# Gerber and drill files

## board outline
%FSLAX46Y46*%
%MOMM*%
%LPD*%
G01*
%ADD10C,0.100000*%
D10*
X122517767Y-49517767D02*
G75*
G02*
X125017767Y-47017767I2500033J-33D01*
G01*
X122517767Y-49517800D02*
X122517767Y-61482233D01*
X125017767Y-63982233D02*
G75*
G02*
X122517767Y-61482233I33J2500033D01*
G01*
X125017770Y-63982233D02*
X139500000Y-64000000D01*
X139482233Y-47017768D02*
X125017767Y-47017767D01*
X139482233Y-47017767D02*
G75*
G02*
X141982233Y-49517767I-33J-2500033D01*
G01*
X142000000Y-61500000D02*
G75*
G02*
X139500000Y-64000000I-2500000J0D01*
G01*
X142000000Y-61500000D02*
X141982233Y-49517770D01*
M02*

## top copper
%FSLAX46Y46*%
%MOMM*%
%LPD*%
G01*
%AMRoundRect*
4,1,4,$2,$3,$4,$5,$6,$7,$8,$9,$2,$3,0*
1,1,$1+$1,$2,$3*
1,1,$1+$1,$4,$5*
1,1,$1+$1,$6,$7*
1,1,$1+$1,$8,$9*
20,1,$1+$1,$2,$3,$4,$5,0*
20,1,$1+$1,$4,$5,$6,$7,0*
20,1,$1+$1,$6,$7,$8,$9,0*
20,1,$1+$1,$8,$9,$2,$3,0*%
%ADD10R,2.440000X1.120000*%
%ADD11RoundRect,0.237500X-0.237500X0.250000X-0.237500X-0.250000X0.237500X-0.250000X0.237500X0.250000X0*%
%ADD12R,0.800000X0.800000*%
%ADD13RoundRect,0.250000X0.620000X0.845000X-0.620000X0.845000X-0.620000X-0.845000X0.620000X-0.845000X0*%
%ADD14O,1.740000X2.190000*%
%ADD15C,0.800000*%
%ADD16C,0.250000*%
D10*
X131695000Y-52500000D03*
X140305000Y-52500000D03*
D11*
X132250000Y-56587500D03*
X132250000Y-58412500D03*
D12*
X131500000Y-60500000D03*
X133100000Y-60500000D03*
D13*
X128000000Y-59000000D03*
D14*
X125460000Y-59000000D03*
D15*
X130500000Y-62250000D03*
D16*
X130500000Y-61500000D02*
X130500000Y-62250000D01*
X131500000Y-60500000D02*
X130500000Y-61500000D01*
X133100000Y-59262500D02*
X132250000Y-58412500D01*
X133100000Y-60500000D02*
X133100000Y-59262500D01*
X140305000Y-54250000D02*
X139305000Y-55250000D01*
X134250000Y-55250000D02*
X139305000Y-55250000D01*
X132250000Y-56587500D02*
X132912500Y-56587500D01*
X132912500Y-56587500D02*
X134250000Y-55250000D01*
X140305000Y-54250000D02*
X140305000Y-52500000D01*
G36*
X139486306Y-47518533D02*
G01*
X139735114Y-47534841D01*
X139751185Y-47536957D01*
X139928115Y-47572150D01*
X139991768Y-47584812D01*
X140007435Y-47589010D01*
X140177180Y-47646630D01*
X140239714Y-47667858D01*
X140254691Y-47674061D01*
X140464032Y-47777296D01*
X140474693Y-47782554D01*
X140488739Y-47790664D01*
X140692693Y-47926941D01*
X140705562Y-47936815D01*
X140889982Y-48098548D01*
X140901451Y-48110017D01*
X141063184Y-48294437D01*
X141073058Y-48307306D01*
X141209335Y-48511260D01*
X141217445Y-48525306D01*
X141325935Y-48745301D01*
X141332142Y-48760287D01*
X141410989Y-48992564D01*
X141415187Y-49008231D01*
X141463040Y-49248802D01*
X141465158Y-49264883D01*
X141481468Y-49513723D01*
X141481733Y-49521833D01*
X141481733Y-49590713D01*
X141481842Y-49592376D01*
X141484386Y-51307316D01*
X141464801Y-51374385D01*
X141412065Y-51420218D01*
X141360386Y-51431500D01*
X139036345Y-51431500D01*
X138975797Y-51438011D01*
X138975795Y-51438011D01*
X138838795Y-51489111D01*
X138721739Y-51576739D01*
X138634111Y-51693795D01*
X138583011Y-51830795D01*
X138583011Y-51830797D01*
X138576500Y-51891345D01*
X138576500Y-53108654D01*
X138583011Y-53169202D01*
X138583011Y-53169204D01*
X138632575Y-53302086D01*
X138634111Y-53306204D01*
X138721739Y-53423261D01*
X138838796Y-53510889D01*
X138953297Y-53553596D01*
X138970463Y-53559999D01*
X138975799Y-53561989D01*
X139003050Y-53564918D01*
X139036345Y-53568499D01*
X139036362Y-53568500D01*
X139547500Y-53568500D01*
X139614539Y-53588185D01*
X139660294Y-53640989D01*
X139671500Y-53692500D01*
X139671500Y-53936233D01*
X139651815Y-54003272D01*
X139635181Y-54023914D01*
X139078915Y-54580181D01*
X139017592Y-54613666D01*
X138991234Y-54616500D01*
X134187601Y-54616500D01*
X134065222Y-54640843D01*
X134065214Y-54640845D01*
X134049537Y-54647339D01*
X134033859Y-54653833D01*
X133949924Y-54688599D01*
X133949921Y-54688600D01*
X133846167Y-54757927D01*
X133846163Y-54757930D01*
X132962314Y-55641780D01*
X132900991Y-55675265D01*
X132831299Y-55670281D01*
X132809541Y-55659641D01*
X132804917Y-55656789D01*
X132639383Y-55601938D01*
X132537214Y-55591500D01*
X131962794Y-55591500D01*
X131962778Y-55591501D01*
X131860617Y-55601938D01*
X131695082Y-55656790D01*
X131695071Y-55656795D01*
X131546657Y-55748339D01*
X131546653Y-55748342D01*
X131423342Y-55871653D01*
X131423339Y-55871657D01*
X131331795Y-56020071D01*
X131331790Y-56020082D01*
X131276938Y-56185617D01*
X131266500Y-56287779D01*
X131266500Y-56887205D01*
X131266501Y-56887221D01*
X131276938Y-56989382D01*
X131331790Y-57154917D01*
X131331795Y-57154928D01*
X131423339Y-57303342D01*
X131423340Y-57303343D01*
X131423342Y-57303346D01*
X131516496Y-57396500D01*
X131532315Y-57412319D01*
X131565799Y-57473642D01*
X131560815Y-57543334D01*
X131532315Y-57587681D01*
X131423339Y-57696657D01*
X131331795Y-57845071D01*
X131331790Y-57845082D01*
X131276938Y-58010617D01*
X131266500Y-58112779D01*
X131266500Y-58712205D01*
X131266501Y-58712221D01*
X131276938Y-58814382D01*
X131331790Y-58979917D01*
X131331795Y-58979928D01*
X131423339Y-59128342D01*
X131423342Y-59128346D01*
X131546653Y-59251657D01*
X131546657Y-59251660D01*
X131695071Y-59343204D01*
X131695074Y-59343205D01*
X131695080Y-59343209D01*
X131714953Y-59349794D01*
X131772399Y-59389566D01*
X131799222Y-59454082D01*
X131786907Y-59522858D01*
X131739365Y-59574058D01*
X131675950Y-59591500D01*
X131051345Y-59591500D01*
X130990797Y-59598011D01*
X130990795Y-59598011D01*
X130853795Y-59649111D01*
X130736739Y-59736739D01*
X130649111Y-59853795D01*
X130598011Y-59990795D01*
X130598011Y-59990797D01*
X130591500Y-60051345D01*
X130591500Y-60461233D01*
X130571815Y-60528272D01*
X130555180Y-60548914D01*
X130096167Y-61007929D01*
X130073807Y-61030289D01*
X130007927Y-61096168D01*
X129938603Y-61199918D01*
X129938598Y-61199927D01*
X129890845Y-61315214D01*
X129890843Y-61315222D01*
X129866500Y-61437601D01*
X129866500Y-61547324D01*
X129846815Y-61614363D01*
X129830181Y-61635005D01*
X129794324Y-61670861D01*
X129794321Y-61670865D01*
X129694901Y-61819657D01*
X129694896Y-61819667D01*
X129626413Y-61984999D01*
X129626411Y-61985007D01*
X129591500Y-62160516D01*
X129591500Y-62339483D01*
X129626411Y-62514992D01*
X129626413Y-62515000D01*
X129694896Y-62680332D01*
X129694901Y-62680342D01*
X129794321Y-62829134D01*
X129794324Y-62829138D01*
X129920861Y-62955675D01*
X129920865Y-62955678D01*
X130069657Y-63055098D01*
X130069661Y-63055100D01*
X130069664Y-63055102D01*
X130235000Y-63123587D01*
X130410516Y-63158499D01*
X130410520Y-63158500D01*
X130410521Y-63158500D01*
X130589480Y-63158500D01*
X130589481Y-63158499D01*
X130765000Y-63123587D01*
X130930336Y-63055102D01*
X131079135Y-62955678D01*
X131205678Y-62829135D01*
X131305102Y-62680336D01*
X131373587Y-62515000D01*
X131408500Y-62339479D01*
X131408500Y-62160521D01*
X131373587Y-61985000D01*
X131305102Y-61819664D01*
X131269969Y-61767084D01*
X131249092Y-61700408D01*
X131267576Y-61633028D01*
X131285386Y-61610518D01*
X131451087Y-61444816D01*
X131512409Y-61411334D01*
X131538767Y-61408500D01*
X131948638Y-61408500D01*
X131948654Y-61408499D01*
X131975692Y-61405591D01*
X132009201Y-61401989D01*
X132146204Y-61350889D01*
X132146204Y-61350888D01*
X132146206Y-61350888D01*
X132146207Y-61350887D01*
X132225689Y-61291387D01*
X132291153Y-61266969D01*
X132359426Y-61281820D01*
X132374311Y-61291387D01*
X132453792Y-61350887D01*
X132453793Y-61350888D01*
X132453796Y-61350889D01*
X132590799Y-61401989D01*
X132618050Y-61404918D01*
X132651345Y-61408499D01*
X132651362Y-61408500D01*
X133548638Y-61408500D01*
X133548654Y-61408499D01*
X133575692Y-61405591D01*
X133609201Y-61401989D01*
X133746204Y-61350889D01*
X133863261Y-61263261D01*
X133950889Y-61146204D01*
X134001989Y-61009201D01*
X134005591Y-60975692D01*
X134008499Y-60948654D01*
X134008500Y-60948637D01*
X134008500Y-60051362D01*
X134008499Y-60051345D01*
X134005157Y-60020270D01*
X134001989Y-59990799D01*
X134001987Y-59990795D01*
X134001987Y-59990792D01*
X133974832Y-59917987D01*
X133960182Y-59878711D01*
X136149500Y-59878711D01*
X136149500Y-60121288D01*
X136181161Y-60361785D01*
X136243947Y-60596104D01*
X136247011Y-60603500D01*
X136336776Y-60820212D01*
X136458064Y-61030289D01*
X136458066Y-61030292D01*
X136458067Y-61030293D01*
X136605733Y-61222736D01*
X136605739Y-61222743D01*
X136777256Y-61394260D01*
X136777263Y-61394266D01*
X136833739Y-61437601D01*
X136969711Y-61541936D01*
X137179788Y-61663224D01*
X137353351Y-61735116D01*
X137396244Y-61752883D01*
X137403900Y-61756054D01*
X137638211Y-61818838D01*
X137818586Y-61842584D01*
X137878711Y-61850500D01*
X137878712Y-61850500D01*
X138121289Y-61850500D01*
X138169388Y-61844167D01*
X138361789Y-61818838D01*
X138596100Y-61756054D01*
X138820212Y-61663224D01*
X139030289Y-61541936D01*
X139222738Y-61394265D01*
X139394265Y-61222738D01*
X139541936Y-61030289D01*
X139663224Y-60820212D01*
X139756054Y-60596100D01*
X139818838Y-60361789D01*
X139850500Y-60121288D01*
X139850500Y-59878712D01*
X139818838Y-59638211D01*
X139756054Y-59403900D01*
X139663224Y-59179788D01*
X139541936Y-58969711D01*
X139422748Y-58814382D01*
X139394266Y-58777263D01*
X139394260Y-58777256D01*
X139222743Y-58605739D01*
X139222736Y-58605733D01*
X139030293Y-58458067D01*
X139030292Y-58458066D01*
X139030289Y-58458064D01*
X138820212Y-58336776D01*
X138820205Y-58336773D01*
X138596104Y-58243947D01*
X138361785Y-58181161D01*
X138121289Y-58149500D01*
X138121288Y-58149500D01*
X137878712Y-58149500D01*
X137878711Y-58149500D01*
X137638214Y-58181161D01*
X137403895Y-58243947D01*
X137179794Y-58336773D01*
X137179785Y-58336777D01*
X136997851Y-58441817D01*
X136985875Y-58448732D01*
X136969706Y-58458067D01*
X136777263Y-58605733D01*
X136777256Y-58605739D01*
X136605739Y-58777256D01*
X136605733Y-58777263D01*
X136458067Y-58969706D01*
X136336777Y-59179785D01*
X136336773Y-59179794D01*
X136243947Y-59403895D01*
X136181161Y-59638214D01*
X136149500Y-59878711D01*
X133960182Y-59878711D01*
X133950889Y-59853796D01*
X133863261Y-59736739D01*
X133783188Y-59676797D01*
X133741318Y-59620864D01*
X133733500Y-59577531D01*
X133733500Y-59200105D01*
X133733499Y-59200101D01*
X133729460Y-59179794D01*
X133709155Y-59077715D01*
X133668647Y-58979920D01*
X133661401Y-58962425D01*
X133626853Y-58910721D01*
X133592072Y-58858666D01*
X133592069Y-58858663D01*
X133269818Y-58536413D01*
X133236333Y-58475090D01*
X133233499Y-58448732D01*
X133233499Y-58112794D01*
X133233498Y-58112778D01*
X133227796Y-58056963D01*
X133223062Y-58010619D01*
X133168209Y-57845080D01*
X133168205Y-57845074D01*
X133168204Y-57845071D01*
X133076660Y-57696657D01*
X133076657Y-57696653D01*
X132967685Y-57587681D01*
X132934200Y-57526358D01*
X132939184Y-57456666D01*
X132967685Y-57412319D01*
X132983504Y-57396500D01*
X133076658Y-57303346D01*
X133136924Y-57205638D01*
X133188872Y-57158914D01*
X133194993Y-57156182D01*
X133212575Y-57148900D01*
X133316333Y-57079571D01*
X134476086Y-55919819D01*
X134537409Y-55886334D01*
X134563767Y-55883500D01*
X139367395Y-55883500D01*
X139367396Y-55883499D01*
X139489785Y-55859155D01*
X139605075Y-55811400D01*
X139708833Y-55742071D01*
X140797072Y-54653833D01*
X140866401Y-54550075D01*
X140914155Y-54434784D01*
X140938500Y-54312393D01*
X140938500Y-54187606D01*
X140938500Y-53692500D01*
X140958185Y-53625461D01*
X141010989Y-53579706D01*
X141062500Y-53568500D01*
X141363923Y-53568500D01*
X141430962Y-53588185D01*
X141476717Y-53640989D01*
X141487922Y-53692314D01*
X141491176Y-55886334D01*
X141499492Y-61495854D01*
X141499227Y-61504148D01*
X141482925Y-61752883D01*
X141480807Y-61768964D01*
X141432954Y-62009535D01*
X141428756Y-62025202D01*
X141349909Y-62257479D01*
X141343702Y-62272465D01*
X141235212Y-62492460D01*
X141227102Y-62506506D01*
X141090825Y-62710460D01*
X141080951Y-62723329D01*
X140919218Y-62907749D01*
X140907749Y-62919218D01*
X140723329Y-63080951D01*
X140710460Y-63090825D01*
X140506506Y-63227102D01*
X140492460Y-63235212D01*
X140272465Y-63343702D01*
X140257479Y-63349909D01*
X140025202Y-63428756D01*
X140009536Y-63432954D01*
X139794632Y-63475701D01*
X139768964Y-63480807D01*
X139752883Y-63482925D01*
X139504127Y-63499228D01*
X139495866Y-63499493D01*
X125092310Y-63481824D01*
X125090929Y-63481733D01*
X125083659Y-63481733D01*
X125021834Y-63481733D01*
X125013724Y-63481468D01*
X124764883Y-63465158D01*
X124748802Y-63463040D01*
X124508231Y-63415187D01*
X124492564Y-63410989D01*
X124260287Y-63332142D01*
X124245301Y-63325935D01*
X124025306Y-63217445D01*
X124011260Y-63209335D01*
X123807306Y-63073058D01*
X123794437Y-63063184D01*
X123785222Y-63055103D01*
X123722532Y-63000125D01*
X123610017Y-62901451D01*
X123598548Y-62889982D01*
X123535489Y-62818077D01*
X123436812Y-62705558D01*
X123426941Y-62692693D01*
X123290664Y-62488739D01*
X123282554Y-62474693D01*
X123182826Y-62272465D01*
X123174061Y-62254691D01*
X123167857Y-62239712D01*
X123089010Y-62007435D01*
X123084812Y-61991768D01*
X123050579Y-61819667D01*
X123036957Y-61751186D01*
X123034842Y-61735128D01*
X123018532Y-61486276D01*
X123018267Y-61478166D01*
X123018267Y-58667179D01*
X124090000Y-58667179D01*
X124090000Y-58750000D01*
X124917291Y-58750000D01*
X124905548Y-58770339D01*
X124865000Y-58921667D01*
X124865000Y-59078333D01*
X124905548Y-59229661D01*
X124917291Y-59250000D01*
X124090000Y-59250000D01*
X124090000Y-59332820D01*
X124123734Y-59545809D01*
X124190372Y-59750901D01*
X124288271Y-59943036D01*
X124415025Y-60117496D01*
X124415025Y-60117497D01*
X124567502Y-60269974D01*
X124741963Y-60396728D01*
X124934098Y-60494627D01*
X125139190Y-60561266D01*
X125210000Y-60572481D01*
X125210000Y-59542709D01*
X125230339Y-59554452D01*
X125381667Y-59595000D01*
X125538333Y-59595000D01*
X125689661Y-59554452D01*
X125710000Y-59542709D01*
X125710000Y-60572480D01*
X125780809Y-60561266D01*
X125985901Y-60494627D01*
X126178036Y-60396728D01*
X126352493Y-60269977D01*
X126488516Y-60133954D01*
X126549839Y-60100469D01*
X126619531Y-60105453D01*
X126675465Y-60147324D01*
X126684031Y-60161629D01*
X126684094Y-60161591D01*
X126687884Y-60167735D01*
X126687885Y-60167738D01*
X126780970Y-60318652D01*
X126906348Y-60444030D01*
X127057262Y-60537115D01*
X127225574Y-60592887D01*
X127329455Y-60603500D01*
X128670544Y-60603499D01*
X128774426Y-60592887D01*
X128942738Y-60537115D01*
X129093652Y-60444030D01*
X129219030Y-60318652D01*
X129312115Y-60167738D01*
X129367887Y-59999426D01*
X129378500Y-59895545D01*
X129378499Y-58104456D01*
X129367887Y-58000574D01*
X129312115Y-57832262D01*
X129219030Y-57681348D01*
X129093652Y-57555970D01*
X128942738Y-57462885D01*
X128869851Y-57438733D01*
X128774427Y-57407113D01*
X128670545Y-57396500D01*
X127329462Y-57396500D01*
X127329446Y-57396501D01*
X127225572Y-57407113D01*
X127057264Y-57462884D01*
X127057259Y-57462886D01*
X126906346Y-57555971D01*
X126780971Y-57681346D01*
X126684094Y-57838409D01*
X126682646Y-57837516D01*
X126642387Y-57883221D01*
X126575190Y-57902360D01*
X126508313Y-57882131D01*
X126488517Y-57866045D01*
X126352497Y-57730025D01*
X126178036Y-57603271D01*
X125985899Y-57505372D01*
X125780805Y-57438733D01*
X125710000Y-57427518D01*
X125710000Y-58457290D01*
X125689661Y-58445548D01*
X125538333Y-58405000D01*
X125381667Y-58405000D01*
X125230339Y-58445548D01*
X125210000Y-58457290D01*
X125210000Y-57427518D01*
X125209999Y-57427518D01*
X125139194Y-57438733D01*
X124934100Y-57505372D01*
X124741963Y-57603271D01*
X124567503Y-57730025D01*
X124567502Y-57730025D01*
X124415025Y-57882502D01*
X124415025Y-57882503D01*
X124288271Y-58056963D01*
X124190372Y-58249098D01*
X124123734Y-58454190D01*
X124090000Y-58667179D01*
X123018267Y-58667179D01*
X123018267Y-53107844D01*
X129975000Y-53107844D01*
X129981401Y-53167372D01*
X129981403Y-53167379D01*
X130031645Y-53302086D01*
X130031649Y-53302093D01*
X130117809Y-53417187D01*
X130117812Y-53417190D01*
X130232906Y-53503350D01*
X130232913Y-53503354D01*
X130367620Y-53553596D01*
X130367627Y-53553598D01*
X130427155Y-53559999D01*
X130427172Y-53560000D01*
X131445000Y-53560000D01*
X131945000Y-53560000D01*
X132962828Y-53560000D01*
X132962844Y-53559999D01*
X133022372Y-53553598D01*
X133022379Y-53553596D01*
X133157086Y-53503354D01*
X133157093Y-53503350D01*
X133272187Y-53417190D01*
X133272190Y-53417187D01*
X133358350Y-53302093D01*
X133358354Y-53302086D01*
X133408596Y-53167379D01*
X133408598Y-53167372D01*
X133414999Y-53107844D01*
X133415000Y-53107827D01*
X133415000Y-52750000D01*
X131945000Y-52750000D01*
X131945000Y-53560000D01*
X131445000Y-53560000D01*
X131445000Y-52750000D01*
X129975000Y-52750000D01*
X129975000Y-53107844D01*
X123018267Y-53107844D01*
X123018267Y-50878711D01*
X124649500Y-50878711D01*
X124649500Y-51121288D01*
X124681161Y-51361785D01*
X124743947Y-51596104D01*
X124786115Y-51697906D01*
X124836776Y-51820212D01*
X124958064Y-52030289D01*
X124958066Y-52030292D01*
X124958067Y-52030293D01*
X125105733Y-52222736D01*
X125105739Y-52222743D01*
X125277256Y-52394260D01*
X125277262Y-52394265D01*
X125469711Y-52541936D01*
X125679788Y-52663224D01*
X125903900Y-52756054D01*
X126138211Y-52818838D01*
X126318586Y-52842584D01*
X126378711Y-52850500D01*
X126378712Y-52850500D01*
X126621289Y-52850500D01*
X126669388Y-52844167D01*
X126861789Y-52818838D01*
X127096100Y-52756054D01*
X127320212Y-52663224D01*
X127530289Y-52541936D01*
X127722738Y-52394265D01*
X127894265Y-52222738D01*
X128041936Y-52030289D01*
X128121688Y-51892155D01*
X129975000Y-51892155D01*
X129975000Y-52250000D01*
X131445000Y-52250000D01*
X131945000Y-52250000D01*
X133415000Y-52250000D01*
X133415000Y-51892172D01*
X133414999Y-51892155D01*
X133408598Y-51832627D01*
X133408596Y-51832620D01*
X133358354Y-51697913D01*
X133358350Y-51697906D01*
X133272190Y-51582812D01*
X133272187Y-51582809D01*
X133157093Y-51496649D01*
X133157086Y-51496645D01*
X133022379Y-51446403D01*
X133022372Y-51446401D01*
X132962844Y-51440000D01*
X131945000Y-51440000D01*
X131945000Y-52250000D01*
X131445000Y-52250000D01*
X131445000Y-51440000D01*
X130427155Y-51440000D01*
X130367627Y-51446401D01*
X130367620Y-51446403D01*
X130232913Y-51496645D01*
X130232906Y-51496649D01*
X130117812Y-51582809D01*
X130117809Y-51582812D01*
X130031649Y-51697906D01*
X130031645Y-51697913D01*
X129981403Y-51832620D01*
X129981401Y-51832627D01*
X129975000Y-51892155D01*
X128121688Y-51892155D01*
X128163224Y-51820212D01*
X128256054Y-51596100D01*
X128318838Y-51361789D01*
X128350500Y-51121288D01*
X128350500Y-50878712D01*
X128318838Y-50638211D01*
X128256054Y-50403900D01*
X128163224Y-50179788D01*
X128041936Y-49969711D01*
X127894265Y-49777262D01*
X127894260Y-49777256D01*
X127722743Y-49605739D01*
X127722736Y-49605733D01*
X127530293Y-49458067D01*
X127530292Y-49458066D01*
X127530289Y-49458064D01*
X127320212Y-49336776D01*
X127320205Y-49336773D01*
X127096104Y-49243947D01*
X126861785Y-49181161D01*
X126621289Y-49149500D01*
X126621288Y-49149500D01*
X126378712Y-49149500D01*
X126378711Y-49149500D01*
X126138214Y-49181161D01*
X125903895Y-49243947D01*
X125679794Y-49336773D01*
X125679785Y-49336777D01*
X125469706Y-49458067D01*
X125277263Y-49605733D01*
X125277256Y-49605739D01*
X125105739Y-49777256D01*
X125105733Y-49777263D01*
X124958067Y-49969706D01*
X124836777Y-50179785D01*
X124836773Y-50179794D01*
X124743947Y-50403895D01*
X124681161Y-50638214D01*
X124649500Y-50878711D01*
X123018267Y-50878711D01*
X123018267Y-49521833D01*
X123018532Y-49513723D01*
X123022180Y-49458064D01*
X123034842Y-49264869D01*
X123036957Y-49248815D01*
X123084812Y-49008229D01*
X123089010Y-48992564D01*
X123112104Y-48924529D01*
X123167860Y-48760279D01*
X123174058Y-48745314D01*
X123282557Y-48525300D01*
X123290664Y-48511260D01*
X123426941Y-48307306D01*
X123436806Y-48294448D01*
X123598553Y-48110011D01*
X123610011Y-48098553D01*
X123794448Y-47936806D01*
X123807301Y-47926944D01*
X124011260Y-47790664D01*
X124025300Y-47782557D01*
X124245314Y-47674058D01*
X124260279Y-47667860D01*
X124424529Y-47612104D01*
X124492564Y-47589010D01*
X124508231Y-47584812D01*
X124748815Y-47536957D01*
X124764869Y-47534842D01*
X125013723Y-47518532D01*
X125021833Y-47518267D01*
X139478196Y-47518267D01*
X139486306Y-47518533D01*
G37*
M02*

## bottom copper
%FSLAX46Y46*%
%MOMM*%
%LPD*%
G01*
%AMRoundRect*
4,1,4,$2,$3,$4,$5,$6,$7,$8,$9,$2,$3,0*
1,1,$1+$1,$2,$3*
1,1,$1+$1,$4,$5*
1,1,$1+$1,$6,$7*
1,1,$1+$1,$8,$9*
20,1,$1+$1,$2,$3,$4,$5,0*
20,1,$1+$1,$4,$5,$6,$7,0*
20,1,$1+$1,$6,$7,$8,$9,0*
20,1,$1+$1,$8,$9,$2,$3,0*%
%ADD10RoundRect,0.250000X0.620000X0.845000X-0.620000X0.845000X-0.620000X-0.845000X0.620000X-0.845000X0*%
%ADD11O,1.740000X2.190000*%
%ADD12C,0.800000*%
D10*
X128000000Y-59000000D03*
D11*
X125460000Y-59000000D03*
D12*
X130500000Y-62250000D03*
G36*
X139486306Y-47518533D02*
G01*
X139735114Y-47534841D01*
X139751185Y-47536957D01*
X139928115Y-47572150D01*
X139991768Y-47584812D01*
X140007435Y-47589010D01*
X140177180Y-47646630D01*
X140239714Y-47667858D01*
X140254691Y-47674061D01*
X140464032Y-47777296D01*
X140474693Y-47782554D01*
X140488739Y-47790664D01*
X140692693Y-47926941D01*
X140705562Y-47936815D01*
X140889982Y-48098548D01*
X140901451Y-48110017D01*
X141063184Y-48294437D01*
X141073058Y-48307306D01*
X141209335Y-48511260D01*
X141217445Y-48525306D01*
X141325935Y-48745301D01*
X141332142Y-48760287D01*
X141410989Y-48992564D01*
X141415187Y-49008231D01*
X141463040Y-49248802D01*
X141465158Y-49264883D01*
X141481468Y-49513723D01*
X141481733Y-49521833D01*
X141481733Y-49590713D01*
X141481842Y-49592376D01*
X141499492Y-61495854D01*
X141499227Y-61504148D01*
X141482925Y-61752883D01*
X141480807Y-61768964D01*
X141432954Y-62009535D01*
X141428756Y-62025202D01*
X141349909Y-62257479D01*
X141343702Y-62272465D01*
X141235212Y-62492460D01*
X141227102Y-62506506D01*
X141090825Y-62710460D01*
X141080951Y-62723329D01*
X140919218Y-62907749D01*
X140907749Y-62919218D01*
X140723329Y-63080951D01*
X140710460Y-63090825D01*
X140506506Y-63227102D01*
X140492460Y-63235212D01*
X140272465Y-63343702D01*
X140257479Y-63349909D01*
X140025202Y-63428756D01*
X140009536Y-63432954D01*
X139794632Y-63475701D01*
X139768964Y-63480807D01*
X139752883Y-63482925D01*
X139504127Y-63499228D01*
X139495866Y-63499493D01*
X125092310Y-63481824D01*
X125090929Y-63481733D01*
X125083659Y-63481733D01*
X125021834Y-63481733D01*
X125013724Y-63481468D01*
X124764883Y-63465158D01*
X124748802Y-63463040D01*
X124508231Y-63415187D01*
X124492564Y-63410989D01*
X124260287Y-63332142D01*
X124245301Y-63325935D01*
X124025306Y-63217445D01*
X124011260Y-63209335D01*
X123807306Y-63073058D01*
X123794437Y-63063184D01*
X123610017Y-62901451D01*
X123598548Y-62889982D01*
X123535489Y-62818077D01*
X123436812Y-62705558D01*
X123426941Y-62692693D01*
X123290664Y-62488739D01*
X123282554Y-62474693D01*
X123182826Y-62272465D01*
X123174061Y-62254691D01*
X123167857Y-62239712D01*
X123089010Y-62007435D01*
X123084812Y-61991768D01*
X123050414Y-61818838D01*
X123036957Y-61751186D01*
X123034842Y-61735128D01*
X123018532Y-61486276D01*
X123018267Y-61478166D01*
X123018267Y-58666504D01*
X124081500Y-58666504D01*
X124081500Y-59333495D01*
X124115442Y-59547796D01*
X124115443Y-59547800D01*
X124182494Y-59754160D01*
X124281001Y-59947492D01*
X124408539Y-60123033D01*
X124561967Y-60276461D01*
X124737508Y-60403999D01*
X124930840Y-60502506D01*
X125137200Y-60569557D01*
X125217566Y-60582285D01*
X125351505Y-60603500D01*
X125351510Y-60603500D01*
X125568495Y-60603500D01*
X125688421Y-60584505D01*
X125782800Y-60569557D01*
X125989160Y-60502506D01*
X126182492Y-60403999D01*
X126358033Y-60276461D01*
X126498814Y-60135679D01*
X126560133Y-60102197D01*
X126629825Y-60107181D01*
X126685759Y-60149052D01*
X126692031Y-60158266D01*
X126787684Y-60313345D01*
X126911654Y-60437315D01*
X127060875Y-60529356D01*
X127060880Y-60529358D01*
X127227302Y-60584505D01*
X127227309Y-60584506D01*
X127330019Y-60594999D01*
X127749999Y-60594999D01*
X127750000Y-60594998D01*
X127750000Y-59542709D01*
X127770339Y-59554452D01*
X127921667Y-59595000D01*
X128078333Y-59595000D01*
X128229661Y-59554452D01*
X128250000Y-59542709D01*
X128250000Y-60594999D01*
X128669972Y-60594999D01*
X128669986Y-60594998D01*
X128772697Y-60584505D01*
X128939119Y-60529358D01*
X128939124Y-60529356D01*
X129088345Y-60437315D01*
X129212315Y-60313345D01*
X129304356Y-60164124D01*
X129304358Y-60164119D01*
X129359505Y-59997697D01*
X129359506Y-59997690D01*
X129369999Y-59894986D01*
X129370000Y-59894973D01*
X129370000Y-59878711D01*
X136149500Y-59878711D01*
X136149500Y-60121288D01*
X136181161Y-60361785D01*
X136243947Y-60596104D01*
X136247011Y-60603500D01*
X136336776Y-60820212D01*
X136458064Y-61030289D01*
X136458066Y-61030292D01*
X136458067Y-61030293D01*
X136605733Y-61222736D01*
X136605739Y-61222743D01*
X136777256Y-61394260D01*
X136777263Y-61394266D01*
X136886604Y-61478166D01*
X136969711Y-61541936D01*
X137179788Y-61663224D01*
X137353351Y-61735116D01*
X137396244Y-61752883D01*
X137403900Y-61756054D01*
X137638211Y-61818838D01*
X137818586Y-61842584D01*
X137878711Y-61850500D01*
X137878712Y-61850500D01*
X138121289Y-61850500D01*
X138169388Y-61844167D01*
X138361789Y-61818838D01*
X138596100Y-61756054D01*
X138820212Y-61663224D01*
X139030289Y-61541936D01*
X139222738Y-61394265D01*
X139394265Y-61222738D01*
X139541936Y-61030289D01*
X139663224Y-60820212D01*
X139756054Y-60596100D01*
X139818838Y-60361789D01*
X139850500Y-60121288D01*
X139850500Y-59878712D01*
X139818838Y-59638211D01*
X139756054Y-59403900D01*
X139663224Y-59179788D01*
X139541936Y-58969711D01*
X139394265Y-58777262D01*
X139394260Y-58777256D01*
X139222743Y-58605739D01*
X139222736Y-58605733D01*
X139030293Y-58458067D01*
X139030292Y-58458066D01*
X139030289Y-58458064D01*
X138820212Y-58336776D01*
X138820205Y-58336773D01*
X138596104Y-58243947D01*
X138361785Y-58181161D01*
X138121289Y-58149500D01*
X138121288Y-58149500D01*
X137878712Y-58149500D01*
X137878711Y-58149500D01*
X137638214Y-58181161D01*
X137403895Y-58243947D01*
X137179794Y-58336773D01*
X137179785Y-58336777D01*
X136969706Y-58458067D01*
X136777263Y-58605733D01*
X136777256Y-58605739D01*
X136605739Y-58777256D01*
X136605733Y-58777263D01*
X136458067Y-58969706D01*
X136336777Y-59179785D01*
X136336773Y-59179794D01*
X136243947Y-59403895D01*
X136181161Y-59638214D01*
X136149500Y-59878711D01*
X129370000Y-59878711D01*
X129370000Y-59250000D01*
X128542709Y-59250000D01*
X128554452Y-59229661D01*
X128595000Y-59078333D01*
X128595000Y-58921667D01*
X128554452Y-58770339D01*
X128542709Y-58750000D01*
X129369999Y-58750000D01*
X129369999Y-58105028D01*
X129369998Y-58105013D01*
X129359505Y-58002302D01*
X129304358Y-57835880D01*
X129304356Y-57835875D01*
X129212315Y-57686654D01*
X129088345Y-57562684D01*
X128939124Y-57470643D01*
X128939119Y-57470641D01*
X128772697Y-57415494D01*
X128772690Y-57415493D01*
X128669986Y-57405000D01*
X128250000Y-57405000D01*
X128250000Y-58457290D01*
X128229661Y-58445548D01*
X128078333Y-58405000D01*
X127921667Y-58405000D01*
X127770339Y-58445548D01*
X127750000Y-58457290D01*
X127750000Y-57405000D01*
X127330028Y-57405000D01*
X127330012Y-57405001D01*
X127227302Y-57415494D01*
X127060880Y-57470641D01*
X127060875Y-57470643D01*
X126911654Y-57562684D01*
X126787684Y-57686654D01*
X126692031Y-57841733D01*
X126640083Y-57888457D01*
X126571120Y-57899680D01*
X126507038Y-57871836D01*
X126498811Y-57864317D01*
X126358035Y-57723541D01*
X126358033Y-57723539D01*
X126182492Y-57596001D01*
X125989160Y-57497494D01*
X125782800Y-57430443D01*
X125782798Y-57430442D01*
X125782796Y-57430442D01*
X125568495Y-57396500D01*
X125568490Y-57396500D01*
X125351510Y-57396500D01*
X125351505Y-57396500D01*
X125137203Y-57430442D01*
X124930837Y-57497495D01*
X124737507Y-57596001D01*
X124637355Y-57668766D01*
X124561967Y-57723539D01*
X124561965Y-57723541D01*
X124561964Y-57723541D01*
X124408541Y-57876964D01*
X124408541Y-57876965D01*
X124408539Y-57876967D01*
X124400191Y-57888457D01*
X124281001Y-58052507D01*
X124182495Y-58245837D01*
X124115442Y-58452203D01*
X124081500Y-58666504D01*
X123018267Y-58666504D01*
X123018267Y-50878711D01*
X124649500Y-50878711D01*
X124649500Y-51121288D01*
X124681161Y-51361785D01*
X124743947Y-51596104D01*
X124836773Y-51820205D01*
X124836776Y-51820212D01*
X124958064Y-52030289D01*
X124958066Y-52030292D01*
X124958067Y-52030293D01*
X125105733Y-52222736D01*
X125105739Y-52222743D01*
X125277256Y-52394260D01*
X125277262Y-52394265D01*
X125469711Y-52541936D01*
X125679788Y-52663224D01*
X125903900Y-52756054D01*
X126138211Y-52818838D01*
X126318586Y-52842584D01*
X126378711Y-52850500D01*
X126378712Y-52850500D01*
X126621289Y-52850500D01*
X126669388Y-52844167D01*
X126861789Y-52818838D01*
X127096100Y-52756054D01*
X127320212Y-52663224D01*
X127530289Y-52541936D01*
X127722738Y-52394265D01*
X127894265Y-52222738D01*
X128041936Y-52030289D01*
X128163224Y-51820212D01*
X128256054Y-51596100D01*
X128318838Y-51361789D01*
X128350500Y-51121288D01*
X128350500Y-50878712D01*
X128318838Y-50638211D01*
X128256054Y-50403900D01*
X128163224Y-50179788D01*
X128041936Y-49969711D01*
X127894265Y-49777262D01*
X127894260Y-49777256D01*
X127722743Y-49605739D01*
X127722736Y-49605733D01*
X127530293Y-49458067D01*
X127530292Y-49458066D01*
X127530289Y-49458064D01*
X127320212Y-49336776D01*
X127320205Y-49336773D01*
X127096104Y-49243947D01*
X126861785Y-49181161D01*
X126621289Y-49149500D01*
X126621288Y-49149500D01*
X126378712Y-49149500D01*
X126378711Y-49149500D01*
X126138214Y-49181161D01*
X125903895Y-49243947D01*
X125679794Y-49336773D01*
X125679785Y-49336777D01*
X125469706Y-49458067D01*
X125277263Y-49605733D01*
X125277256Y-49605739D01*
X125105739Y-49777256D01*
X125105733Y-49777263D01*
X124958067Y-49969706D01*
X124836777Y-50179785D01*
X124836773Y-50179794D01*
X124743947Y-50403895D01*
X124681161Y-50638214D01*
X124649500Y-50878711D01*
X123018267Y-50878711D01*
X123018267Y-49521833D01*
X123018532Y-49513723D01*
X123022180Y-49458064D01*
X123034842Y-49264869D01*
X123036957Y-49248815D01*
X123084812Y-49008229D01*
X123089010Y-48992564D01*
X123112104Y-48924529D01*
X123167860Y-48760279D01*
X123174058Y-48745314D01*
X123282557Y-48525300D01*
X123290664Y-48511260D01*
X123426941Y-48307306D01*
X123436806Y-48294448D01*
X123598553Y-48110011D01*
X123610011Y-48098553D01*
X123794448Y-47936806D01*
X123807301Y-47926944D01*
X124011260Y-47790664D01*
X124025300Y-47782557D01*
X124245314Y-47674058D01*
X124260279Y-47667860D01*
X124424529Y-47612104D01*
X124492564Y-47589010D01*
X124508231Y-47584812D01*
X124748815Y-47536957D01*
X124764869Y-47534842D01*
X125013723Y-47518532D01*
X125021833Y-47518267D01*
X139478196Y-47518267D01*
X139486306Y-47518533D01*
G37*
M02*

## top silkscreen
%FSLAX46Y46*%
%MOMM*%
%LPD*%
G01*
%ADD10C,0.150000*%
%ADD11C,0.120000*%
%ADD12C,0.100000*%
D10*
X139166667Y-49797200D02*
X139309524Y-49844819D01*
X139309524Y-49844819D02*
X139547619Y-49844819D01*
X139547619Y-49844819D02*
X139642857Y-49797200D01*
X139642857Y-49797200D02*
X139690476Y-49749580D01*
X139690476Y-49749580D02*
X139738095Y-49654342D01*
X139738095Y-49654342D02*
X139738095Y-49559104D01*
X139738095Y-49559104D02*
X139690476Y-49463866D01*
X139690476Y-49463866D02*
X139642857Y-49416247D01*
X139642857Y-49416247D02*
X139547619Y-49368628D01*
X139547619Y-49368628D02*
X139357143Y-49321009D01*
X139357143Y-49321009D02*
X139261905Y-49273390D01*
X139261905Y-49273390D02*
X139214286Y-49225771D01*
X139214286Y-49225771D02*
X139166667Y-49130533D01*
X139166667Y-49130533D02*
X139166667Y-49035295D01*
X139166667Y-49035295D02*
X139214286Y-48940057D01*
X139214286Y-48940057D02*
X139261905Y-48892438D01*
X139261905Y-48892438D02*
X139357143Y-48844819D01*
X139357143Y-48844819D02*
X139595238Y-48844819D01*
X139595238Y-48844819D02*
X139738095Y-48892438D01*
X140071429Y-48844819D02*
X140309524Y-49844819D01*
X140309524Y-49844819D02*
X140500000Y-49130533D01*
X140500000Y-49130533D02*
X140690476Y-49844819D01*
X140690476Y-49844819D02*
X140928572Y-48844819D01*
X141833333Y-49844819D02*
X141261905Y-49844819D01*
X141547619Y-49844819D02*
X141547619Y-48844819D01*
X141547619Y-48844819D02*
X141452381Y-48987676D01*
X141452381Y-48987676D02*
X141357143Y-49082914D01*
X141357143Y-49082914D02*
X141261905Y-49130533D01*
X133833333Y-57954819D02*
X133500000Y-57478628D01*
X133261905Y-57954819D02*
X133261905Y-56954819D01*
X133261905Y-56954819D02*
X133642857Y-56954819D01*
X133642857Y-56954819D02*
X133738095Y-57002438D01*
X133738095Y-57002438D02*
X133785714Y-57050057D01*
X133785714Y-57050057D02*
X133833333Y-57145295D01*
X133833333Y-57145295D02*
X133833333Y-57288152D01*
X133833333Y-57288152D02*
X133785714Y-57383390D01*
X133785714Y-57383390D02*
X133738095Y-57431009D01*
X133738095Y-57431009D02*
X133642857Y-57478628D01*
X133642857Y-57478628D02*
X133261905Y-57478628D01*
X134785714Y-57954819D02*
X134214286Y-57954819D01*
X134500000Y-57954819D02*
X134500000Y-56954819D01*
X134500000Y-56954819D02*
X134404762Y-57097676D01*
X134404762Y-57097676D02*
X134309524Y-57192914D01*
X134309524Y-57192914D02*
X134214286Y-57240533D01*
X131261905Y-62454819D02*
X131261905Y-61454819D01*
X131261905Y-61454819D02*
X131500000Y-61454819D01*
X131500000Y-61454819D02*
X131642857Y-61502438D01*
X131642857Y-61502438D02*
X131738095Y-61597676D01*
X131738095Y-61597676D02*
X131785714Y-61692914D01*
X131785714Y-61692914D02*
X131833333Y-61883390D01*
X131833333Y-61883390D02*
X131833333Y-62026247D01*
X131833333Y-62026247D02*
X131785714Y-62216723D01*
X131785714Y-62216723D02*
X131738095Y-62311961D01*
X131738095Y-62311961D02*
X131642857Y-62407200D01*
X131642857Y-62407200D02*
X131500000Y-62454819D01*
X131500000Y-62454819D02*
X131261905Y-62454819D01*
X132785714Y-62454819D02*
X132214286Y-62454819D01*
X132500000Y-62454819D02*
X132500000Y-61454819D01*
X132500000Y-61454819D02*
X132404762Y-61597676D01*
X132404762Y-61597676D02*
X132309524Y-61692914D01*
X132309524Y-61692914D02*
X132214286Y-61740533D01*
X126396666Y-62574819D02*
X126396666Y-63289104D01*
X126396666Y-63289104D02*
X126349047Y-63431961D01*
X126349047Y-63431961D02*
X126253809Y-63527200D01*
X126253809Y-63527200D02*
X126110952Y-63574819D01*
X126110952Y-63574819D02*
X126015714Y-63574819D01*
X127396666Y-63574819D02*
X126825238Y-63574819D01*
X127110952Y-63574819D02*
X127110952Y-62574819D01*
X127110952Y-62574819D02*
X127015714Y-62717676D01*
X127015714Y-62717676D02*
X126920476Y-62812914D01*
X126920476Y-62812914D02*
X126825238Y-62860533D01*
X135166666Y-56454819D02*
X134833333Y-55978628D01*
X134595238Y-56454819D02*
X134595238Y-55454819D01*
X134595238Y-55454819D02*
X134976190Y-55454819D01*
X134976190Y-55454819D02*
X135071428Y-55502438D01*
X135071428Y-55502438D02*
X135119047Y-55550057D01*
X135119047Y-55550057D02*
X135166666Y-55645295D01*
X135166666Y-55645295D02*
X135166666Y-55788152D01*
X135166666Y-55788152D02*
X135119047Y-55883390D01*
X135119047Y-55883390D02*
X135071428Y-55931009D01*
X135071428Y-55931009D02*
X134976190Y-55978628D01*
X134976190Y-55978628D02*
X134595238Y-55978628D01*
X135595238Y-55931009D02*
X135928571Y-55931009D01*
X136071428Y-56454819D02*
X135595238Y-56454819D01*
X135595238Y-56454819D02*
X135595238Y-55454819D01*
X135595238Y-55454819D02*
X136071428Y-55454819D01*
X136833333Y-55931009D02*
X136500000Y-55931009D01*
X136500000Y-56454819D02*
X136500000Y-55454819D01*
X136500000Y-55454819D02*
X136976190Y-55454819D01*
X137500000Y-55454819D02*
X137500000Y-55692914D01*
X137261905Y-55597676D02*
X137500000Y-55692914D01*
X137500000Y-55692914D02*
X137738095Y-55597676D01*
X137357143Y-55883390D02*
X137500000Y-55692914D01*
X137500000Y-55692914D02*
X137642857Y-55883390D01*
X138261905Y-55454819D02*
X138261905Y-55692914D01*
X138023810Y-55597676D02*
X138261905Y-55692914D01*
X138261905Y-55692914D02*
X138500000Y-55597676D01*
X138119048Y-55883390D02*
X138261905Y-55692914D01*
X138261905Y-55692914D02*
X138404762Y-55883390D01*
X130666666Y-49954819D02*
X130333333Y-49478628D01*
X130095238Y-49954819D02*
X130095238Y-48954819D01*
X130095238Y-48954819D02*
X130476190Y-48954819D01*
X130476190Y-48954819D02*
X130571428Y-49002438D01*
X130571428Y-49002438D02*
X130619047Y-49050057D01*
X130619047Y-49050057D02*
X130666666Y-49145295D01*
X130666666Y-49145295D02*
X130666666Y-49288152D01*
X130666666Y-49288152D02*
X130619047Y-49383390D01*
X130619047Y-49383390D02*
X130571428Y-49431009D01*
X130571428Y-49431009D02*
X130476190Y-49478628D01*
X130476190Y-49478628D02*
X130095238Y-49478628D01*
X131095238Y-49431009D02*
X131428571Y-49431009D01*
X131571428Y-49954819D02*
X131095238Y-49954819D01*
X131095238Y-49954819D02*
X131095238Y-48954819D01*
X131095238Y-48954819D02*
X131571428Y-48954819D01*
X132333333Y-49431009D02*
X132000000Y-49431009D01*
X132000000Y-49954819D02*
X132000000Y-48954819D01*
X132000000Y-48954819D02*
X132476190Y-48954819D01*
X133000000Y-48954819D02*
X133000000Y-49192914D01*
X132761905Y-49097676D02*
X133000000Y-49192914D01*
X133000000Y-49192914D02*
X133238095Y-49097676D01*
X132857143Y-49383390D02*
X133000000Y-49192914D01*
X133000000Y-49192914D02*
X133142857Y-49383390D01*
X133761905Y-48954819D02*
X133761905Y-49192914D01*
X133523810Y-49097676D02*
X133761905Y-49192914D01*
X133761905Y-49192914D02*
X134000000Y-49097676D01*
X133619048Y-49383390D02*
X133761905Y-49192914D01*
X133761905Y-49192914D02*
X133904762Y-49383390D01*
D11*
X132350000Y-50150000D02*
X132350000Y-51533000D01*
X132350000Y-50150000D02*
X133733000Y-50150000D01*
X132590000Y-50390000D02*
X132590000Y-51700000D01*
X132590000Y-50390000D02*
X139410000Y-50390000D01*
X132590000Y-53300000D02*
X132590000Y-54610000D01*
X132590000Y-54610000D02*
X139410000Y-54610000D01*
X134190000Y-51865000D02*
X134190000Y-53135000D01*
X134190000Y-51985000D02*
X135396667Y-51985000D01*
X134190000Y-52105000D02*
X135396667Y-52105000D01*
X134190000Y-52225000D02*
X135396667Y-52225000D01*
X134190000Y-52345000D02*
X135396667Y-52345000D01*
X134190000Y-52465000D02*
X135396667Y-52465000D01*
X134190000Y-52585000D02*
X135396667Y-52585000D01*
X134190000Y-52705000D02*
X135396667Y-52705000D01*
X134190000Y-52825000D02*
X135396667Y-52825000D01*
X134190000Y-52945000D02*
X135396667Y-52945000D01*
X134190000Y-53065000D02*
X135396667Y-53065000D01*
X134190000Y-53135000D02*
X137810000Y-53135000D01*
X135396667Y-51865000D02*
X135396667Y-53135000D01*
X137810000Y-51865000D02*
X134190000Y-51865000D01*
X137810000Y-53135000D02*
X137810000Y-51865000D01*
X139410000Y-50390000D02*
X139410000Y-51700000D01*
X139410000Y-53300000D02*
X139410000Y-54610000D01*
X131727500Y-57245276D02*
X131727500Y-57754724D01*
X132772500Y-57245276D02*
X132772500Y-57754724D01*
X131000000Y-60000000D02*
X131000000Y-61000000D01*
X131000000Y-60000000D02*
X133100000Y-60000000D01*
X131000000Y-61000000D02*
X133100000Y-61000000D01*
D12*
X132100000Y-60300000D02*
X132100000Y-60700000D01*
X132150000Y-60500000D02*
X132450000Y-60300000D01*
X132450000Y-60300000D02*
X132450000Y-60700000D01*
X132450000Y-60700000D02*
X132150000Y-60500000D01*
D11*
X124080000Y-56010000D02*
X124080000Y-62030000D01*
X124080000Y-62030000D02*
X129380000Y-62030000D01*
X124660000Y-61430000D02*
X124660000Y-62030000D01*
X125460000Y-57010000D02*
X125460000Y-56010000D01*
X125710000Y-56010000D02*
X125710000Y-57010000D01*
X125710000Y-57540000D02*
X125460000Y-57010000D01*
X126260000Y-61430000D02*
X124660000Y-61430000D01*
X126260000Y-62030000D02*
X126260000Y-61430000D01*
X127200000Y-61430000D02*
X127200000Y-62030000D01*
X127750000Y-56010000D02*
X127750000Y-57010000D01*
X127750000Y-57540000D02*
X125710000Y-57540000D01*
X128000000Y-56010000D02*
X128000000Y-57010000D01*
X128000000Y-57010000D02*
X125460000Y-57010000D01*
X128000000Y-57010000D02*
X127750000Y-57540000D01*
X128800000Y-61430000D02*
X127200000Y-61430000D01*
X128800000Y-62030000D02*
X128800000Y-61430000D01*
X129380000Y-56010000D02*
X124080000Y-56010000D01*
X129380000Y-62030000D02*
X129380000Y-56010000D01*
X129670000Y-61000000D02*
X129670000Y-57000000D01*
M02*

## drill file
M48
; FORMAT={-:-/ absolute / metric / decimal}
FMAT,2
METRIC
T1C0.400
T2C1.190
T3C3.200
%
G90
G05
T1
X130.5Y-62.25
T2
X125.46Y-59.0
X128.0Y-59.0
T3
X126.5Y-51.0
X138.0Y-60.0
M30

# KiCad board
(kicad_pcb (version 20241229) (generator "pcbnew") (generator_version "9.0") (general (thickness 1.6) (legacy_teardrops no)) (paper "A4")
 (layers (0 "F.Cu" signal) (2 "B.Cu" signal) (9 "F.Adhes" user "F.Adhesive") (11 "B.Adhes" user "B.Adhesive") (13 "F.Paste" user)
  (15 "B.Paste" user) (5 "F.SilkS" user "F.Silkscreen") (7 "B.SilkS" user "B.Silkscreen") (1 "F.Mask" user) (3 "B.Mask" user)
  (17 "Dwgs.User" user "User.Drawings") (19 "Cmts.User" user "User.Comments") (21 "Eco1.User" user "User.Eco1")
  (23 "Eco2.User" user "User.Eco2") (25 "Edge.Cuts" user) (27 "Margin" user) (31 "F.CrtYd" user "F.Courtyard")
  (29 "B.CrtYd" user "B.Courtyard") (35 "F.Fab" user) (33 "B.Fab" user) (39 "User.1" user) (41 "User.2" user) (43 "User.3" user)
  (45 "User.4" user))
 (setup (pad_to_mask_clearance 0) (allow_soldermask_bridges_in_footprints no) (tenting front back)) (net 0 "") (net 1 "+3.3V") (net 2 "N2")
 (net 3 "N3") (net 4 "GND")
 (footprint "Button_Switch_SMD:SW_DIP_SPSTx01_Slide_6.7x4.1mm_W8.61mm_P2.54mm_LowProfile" (layer "F.Cu") (at 136 52.5)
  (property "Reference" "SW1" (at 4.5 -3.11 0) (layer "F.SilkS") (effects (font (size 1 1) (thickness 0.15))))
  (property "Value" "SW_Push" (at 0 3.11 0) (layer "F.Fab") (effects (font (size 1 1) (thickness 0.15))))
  (fp_line (start -3.65 -2.35) (end -3.65 -0.967) (stroke (width 0.12) (type solid)) (layer "F.SilkS"))
  (fp_line (start -3.65 -2.35) (end -2.267 -2.35) (stroke (width 0.12) (type solid)) (layer "F.SilkS"))
  (fp_line (start -3.41 -2.11) (end -3.41 -0.8) (stroke (width 0.12) (type solid)) (layer "F.SilkS"))
  (fp_line (start -3.41 -2.11) (end 3.41 -2.11) (stroke (width 0.12) (type solid)) (layer "F.SilkS"))
  (fp_line (start -3.41 0.8) (end -3.41 2.11) (stroke (width 0.12) (type solid)) (layer "F.SilkS"))
  (fp_line (start -3.41 2.11) (end 3.41 2.11) (stroke (width 0.12) (type solid)) (layer "F.SilkS"))
  (fp_line (start -1.81 -0.635) (end -1.81 0.635) (stroke (width 0.12) (type solid)) (layer "F.SilkS"))
  (fp_line (start -1.81 -0.515) (end -0.603333 -0.515) (stroke (width 0.12) (type solid)) (layer "F.SilkS"))
  (fp_line (start -1.81 -0.395) (end -0.603333 -0.395) (stroke (width 0.12) (type solid)) (layer "F.SilkS"))
  (fp_line (start -1.81 -0.275) (end -0.603333 -0.275) (stroke (width 0.12) (type solid)) (layer "F.SilkS"))
  (fp_line (start -1.81 -0.155) (end -0.603333 -0.155) (stroke (width 0.12) (type solid)) (layer "F.SilkS"))
  (fp_line (start -1.81 -0.035) (end -0.603333 -0.035) (stroke (width 0.12) (type solid)) (layer "F.SilkS"))
  (fp_line (start -1.81 0.085) (end -0.603333 0.085) (stroke (width 0.12) (type solid)) (layer "F.SilkS"))
  (fp_line (start -1.81 0.205) (end -0.603333 0.205) (stroke (width 0.12) (type solid)) (layer "F.SilkS"))
  (fp_line (start -1.81 0.325) (end -0.603333 0.325) (stroke (width 0.12) (type solid)) (layer "F.SilkS"))
  (fp_line (start -1.81 0.445) (end -0.603333 0.445) (stroke (width 0.12) (type solid)) (layer "F.SilkS"))
  (fp_line (start -1.81 0.565) (end -0.603333 0.565) (stroke (width 0.12) (type solid)) (layer "F.SilkS"))
  (fp_line (start -1.81 0.635) (end 1.81 0.635) (stroke (width 0.12) (type solid)) (layer "F.SilkS"))
  (fp_line (start -0.603333 -0.635) (end -0.603333 0.635) (stroke (width 0.12) (type solid)) (layer "F.SilkS"))
  (fp_line (start 1.81 -0.635) (end -1.81 -0.635) (stroke (width 0.12) (type solid)) (layer "F.SilkS"))
  (fp_line (start 1.81 0.635) (end 1.81 -0.635) (stroke (width 0.12) (type solid)) (layer "F.SilkS"))
  (fp_line (start 3.41 -2.11) (end 3.41 -0.8) (stroke (width 0.12) (type solid)) (layer "F.SilkS"))
  (fp_line (start 3.41 0.8) (end 3.41 2.11) (stroke (width 0.12) (type solid)) (layer "F.SilkS"))
  (pad "1" smd rect (at -4.305 0) (size 2.44 1.12) (layers "F.Cu" "F.Mask" "F.Paste") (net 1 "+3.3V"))
  (pad "2" smd rect (at 4.305 0) (size 2.44 1.12) (layers "F.Cu" "F.Mask" "F.Paste") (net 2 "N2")))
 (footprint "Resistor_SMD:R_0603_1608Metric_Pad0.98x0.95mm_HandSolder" (layer "F.Cu") (at 132.25 57.5 -90)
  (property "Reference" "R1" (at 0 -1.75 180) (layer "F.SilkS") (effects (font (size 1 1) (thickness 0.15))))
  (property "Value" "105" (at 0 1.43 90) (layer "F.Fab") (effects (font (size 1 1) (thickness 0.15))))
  (fp_line (start -0.254724 0.5225) (end 0.254724 0.5225) (stroke (width 0.12) (type solid)) (layer "F.SilkS"))
  (fp_line (start -0.254724 -0.5225) (end 0.254724 -0.5225) (stroke (width 0.12) (type solid)) (layer "F.SilkS"))
  (pad "1" smd roundrect (at -0.9125 0 270) (size 0.975 0.95) (layers "F.Cu" "F.Mask" "F.Paste") (roundrect_rratio 0.25) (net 2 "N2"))
  (pad "2" smd roundrect (at 0.9125 0 270) (size 0.975 0.95) (layers "F.Cu" "F.Mask" "F.Paste") (roundrect_rratio 0.25) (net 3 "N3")))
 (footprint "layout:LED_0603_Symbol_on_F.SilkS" (layer "F.Cu") (at 132.3 60.5)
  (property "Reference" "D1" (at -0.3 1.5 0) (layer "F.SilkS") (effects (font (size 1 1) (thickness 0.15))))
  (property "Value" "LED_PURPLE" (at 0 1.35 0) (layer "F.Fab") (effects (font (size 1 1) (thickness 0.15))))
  (fp_line (start -1.3 -0.5) (end -1.3 0.5) (stroke (width 0.12) (type solid)) (layer "F.SilkS"))
  (fp_line (start -1.3 -0.5) (end 0.8 -0.5) (stroke (width 0.12) (type solid)) (layer "F.SilkS"))
  (fp_line (start -1.3 0.5) (end 0.8 0.5) (stroke (width 0.12) (type solid)) (layer "F.SilkS"))
  (fp_line (start -0.2 -0.2) (end -0.2 0.2) (stroke (width 0.1) (type solid)) (layer "F.SilkS"))
  (fp_line (start -0.15 0) (end 0.15 -0.2) (stroke (width 0.1) (type solid)) (layer "F.SilkS"))
  (fp_line (start 0.15 -0.2) (end 0.15 0.2) (stroke (width 0.1) (type solid)) (layer "F.SilkS"))
  (fp_line (start 0.15 0.2) (end -0.15 0) (stroke (width 0.1) (type solid)) (layer "F.SilkS"))
  (pad "1" smd rect (at -0.8 0 180) (size 0.8 0.8) (layers "F.Cu" "F.Mask" "F.Paste") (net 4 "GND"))
  (pad "2" smd rect (at 0.8 0 180) (size 0.8 0.8) (layers "F.Cu" "F.Mask" "F.Paste") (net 3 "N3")))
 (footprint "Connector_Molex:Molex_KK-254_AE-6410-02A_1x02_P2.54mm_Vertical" (layer "F.Cu") (at 128 59 180)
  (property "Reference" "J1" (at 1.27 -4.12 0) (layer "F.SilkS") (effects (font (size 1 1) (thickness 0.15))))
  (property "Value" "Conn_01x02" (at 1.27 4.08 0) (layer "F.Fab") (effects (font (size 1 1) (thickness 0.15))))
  (fp_line (start 3.92 2.99) (end 3.92 -3.03) (stroke (width 0.12) (type solid)) (layer "F.SilkS"))
  (fp_line (start 3.92 -3.03) (end -1.38 -3.03) (stroke (width 0.12) (type solid)) (layer "F.SilkS"))
  (fp_line (start 3.34 -2.43) (end 3.34 -3.03) (stroke (width 0.12) (type solid)) (layer "F.SilkS"))
  (fp_line (start 2.54 1.99) (end 2.54 2.99) (stroke (width 0.12) (type solid)) (layer "F.SilkS"))
  (fp_line (start 2.29 2.99) (end 2.29 1.99) (stroke (width 0.12) (type solid)) (layer "F.SilkS"))
  (fp_line (start 2.29 1.46) (end 2.54 1.99) (stroke (width 0.12) (type solid)) (layer "F.SilkS"))
  (fp_line (start 1.74 -2.43) (end 3.34 -2.43) (stroke (width 0.12) (type solid)) (layer "F.SilkS"))
  (fp_line (start 1.74 -3.03) (end 1.74 -2.43) (stroke (width 0.12) (type solid)) (layer "F.SilkS"))
  (fp_line (start 0.8 -2.43) (end 0.8 -3.03) (stroke (width 0.12) (type solid)) (layer "F.SilkS"))
  (fp_line (start 0.25 2.99) (end 0.25 1.99) (stroke (width 0.12) (type solid)) (layer "F.SilkS"))
  (fp_line (start 0.25 1.46) (end 2.29 1.46) (stroke (width 0.12) (type solid)) (layer "F.SilkS"))
  (fp_line (start 0 2.99) (end 0 1.99) (stroke (width 0.12) (type solid)) (layer "F.SilkS"))
  (fp_line (start 0 1.99) (end 2.54 1.99) (stroke (width 0.12) (type solid)) (layer "F.SilkS"))
  (fp_line (start 0 1.99) (end 0.25 1.46) (stroke (width 0.12) (type solid)) (layer "F.SilkS"))
  (fp_line (start -0.8 -2.43) (end 0.8 -2.43) (stroke (width 0.12) (type solid)) (layer "F.SilkS"))
  (fp_line (start -0.8 -3.03) (end -0.8 -2.43) (stroke (width 0.12) (type solid)) (layer "F.SilkS"))
  (fp_line (start -1.38 2.99) (end 3.92 2.99) (stroke (width 0.12) (type solid)) (layer "F.SilkS"))
  (fp_line (start -1.38 -3.03) (end -1.38 2.99) (stroke (width 0.12) (type solid)) (layer "F.SilkS"))
  (fp_line (start -1.67 -2) (end -1.67 2) (stroke (width 0.12) (type solid)) (layer "F.SilkS"))
  (pad "1" thru_hole roundrect (at 0 0 180) (size 1.74 2.19) (drill 1.19) (layers "*.Cu" "*.Mask") (remove_unused_layers no)
   (roundrect_rratio 0.143678) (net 4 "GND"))
  (pad "2" thru_hole oval (at 2.54 0 180) (size 1.74 2.19) (drill 1.19) (layers "*.Cu" "*.Mask") (remove_unused_layers no) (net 1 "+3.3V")))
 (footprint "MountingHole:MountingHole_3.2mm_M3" (layer "F.Cu") (at 138 60)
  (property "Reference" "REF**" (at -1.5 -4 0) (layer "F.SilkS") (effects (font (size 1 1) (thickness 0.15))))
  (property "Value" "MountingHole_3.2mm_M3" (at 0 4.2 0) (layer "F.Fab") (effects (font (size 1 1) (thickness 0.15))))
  (pad "" np_thru_hole circle (at 0 0) (size 3.2 3.2) (drill 3.2) (layers "*.Cu" "*.Mask")))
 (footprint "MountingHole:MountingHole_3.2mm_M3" (layer "F.Cu") (at 126.5 51)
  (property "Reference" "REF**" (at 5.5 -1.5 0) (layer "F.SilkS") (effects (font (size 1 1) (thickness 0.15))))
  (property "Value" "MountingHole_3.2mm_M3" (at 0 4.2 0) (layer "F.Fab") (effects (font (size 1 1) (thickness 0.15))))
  (pad "" np_thru_hole circle (at 0 0) (size 3.2 3.2) (drill 3.2) (layers "*.Cu" "*.Mask")))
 (gr_arc (start 122.517767 49.517767) (mid 123.25 47.75) (end 125.017767 47.017767) (stroke (width 0.1) (type default)) (layer "Edge.Cuts"))
 (gr_line (start 122.517767 49.5178) (end 122.517767 61.482233) (stroke (width 0.1) (type default)) (layer "Edge.Cuts"))
 (gr_arc (start 125.017767 63.982233) (mid 123.25 63.25) (end 122.517767 61.482233) (stroke (width 0.1) (type default)) (layer "Edge.Cuts"))
 (gr_line (start 125.01777 63.982233) (end 139.5 64) (stroke (width 0.1) (type default)) (layer "Edge.Cuts"))
 (gr_line (start 139.482233 47.017768) (end 125.017767 47.017767) (stroke (width 0.1) (type default)) (layer "Edge.Cuts"))
 (gr_arc (start 139.482233 47.017767) (mid 141.25 47.75) (end 141.982233 49.517767) (stroke (width 0.1) (type default)) (layer "Edge.Cuts"))
 (gr_arc (start 142 61.5) (mid 141.267767 63.267767) (end 139.5 64) (stroke (width 0.1) (type default)) (layer "Edge.Cuts"))
 (gr_line (start 142 61.5) (end 141.982233 49.51777) (stroke (width 0.1) (type default)) (layer "Edge.Cuts"))
 (segment (start 130.5 61.5) (end 130.5 62.25) (width 0.25) (layer "F.Cu") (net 4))
 (segment (start 131.5 60.5) (end 130.5 61.5) (width 0.25) (layer "F.Cu") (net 4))
 (via (at 130.5 62.25) (size 0.8) (drill 0.4) (layers "F.Cu" "B.Cu") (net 4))
 (segment (start 133.1 59.2625) (end 132.25 58.4125) (width 0.25) (layer "F.Cu") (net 3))
 (segment (start 133.1 60.5) (end 133.1 59.2625) (width 0.25) (layer "F.Cu") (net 3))
 (segment (start 140.305 54.25) (end 139.305 55.25) (width 0.25) (layer "F.Cu") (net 2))
 (segment (start 134.25 55.25) (end 139.305 55.25) (width 0.25) (layer "F.Cu") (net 2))
 (segment (start 132.25 56.5875) (end 132.9125 56.5875) (width 0.25) (layer "F.Cu") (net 2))
 (segment (start 132.9125 56.5875) (end 134.25 55.25) (width 0.25) (layer "F.Cu") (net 2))
 (segment (start 140.305 54.25) (end 140.305 52.5) (width 0.25) (layer "F.Cu") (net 2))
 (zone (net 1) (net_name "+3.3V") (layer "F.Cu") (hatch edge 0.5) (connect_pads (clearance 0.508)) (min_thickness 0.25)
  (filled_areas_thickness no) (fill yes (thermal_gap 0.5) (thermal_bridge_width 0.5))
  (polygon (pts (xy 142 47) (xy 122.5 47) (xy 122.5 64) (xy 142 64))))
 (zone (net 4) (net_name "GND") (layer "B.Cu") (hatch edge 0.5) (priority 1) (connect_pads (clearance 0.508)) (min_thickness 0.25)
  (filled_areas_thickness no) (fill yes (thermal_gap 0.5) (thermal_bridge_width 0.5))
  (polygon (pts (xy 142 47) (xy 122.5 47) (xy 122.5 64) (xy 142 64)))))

